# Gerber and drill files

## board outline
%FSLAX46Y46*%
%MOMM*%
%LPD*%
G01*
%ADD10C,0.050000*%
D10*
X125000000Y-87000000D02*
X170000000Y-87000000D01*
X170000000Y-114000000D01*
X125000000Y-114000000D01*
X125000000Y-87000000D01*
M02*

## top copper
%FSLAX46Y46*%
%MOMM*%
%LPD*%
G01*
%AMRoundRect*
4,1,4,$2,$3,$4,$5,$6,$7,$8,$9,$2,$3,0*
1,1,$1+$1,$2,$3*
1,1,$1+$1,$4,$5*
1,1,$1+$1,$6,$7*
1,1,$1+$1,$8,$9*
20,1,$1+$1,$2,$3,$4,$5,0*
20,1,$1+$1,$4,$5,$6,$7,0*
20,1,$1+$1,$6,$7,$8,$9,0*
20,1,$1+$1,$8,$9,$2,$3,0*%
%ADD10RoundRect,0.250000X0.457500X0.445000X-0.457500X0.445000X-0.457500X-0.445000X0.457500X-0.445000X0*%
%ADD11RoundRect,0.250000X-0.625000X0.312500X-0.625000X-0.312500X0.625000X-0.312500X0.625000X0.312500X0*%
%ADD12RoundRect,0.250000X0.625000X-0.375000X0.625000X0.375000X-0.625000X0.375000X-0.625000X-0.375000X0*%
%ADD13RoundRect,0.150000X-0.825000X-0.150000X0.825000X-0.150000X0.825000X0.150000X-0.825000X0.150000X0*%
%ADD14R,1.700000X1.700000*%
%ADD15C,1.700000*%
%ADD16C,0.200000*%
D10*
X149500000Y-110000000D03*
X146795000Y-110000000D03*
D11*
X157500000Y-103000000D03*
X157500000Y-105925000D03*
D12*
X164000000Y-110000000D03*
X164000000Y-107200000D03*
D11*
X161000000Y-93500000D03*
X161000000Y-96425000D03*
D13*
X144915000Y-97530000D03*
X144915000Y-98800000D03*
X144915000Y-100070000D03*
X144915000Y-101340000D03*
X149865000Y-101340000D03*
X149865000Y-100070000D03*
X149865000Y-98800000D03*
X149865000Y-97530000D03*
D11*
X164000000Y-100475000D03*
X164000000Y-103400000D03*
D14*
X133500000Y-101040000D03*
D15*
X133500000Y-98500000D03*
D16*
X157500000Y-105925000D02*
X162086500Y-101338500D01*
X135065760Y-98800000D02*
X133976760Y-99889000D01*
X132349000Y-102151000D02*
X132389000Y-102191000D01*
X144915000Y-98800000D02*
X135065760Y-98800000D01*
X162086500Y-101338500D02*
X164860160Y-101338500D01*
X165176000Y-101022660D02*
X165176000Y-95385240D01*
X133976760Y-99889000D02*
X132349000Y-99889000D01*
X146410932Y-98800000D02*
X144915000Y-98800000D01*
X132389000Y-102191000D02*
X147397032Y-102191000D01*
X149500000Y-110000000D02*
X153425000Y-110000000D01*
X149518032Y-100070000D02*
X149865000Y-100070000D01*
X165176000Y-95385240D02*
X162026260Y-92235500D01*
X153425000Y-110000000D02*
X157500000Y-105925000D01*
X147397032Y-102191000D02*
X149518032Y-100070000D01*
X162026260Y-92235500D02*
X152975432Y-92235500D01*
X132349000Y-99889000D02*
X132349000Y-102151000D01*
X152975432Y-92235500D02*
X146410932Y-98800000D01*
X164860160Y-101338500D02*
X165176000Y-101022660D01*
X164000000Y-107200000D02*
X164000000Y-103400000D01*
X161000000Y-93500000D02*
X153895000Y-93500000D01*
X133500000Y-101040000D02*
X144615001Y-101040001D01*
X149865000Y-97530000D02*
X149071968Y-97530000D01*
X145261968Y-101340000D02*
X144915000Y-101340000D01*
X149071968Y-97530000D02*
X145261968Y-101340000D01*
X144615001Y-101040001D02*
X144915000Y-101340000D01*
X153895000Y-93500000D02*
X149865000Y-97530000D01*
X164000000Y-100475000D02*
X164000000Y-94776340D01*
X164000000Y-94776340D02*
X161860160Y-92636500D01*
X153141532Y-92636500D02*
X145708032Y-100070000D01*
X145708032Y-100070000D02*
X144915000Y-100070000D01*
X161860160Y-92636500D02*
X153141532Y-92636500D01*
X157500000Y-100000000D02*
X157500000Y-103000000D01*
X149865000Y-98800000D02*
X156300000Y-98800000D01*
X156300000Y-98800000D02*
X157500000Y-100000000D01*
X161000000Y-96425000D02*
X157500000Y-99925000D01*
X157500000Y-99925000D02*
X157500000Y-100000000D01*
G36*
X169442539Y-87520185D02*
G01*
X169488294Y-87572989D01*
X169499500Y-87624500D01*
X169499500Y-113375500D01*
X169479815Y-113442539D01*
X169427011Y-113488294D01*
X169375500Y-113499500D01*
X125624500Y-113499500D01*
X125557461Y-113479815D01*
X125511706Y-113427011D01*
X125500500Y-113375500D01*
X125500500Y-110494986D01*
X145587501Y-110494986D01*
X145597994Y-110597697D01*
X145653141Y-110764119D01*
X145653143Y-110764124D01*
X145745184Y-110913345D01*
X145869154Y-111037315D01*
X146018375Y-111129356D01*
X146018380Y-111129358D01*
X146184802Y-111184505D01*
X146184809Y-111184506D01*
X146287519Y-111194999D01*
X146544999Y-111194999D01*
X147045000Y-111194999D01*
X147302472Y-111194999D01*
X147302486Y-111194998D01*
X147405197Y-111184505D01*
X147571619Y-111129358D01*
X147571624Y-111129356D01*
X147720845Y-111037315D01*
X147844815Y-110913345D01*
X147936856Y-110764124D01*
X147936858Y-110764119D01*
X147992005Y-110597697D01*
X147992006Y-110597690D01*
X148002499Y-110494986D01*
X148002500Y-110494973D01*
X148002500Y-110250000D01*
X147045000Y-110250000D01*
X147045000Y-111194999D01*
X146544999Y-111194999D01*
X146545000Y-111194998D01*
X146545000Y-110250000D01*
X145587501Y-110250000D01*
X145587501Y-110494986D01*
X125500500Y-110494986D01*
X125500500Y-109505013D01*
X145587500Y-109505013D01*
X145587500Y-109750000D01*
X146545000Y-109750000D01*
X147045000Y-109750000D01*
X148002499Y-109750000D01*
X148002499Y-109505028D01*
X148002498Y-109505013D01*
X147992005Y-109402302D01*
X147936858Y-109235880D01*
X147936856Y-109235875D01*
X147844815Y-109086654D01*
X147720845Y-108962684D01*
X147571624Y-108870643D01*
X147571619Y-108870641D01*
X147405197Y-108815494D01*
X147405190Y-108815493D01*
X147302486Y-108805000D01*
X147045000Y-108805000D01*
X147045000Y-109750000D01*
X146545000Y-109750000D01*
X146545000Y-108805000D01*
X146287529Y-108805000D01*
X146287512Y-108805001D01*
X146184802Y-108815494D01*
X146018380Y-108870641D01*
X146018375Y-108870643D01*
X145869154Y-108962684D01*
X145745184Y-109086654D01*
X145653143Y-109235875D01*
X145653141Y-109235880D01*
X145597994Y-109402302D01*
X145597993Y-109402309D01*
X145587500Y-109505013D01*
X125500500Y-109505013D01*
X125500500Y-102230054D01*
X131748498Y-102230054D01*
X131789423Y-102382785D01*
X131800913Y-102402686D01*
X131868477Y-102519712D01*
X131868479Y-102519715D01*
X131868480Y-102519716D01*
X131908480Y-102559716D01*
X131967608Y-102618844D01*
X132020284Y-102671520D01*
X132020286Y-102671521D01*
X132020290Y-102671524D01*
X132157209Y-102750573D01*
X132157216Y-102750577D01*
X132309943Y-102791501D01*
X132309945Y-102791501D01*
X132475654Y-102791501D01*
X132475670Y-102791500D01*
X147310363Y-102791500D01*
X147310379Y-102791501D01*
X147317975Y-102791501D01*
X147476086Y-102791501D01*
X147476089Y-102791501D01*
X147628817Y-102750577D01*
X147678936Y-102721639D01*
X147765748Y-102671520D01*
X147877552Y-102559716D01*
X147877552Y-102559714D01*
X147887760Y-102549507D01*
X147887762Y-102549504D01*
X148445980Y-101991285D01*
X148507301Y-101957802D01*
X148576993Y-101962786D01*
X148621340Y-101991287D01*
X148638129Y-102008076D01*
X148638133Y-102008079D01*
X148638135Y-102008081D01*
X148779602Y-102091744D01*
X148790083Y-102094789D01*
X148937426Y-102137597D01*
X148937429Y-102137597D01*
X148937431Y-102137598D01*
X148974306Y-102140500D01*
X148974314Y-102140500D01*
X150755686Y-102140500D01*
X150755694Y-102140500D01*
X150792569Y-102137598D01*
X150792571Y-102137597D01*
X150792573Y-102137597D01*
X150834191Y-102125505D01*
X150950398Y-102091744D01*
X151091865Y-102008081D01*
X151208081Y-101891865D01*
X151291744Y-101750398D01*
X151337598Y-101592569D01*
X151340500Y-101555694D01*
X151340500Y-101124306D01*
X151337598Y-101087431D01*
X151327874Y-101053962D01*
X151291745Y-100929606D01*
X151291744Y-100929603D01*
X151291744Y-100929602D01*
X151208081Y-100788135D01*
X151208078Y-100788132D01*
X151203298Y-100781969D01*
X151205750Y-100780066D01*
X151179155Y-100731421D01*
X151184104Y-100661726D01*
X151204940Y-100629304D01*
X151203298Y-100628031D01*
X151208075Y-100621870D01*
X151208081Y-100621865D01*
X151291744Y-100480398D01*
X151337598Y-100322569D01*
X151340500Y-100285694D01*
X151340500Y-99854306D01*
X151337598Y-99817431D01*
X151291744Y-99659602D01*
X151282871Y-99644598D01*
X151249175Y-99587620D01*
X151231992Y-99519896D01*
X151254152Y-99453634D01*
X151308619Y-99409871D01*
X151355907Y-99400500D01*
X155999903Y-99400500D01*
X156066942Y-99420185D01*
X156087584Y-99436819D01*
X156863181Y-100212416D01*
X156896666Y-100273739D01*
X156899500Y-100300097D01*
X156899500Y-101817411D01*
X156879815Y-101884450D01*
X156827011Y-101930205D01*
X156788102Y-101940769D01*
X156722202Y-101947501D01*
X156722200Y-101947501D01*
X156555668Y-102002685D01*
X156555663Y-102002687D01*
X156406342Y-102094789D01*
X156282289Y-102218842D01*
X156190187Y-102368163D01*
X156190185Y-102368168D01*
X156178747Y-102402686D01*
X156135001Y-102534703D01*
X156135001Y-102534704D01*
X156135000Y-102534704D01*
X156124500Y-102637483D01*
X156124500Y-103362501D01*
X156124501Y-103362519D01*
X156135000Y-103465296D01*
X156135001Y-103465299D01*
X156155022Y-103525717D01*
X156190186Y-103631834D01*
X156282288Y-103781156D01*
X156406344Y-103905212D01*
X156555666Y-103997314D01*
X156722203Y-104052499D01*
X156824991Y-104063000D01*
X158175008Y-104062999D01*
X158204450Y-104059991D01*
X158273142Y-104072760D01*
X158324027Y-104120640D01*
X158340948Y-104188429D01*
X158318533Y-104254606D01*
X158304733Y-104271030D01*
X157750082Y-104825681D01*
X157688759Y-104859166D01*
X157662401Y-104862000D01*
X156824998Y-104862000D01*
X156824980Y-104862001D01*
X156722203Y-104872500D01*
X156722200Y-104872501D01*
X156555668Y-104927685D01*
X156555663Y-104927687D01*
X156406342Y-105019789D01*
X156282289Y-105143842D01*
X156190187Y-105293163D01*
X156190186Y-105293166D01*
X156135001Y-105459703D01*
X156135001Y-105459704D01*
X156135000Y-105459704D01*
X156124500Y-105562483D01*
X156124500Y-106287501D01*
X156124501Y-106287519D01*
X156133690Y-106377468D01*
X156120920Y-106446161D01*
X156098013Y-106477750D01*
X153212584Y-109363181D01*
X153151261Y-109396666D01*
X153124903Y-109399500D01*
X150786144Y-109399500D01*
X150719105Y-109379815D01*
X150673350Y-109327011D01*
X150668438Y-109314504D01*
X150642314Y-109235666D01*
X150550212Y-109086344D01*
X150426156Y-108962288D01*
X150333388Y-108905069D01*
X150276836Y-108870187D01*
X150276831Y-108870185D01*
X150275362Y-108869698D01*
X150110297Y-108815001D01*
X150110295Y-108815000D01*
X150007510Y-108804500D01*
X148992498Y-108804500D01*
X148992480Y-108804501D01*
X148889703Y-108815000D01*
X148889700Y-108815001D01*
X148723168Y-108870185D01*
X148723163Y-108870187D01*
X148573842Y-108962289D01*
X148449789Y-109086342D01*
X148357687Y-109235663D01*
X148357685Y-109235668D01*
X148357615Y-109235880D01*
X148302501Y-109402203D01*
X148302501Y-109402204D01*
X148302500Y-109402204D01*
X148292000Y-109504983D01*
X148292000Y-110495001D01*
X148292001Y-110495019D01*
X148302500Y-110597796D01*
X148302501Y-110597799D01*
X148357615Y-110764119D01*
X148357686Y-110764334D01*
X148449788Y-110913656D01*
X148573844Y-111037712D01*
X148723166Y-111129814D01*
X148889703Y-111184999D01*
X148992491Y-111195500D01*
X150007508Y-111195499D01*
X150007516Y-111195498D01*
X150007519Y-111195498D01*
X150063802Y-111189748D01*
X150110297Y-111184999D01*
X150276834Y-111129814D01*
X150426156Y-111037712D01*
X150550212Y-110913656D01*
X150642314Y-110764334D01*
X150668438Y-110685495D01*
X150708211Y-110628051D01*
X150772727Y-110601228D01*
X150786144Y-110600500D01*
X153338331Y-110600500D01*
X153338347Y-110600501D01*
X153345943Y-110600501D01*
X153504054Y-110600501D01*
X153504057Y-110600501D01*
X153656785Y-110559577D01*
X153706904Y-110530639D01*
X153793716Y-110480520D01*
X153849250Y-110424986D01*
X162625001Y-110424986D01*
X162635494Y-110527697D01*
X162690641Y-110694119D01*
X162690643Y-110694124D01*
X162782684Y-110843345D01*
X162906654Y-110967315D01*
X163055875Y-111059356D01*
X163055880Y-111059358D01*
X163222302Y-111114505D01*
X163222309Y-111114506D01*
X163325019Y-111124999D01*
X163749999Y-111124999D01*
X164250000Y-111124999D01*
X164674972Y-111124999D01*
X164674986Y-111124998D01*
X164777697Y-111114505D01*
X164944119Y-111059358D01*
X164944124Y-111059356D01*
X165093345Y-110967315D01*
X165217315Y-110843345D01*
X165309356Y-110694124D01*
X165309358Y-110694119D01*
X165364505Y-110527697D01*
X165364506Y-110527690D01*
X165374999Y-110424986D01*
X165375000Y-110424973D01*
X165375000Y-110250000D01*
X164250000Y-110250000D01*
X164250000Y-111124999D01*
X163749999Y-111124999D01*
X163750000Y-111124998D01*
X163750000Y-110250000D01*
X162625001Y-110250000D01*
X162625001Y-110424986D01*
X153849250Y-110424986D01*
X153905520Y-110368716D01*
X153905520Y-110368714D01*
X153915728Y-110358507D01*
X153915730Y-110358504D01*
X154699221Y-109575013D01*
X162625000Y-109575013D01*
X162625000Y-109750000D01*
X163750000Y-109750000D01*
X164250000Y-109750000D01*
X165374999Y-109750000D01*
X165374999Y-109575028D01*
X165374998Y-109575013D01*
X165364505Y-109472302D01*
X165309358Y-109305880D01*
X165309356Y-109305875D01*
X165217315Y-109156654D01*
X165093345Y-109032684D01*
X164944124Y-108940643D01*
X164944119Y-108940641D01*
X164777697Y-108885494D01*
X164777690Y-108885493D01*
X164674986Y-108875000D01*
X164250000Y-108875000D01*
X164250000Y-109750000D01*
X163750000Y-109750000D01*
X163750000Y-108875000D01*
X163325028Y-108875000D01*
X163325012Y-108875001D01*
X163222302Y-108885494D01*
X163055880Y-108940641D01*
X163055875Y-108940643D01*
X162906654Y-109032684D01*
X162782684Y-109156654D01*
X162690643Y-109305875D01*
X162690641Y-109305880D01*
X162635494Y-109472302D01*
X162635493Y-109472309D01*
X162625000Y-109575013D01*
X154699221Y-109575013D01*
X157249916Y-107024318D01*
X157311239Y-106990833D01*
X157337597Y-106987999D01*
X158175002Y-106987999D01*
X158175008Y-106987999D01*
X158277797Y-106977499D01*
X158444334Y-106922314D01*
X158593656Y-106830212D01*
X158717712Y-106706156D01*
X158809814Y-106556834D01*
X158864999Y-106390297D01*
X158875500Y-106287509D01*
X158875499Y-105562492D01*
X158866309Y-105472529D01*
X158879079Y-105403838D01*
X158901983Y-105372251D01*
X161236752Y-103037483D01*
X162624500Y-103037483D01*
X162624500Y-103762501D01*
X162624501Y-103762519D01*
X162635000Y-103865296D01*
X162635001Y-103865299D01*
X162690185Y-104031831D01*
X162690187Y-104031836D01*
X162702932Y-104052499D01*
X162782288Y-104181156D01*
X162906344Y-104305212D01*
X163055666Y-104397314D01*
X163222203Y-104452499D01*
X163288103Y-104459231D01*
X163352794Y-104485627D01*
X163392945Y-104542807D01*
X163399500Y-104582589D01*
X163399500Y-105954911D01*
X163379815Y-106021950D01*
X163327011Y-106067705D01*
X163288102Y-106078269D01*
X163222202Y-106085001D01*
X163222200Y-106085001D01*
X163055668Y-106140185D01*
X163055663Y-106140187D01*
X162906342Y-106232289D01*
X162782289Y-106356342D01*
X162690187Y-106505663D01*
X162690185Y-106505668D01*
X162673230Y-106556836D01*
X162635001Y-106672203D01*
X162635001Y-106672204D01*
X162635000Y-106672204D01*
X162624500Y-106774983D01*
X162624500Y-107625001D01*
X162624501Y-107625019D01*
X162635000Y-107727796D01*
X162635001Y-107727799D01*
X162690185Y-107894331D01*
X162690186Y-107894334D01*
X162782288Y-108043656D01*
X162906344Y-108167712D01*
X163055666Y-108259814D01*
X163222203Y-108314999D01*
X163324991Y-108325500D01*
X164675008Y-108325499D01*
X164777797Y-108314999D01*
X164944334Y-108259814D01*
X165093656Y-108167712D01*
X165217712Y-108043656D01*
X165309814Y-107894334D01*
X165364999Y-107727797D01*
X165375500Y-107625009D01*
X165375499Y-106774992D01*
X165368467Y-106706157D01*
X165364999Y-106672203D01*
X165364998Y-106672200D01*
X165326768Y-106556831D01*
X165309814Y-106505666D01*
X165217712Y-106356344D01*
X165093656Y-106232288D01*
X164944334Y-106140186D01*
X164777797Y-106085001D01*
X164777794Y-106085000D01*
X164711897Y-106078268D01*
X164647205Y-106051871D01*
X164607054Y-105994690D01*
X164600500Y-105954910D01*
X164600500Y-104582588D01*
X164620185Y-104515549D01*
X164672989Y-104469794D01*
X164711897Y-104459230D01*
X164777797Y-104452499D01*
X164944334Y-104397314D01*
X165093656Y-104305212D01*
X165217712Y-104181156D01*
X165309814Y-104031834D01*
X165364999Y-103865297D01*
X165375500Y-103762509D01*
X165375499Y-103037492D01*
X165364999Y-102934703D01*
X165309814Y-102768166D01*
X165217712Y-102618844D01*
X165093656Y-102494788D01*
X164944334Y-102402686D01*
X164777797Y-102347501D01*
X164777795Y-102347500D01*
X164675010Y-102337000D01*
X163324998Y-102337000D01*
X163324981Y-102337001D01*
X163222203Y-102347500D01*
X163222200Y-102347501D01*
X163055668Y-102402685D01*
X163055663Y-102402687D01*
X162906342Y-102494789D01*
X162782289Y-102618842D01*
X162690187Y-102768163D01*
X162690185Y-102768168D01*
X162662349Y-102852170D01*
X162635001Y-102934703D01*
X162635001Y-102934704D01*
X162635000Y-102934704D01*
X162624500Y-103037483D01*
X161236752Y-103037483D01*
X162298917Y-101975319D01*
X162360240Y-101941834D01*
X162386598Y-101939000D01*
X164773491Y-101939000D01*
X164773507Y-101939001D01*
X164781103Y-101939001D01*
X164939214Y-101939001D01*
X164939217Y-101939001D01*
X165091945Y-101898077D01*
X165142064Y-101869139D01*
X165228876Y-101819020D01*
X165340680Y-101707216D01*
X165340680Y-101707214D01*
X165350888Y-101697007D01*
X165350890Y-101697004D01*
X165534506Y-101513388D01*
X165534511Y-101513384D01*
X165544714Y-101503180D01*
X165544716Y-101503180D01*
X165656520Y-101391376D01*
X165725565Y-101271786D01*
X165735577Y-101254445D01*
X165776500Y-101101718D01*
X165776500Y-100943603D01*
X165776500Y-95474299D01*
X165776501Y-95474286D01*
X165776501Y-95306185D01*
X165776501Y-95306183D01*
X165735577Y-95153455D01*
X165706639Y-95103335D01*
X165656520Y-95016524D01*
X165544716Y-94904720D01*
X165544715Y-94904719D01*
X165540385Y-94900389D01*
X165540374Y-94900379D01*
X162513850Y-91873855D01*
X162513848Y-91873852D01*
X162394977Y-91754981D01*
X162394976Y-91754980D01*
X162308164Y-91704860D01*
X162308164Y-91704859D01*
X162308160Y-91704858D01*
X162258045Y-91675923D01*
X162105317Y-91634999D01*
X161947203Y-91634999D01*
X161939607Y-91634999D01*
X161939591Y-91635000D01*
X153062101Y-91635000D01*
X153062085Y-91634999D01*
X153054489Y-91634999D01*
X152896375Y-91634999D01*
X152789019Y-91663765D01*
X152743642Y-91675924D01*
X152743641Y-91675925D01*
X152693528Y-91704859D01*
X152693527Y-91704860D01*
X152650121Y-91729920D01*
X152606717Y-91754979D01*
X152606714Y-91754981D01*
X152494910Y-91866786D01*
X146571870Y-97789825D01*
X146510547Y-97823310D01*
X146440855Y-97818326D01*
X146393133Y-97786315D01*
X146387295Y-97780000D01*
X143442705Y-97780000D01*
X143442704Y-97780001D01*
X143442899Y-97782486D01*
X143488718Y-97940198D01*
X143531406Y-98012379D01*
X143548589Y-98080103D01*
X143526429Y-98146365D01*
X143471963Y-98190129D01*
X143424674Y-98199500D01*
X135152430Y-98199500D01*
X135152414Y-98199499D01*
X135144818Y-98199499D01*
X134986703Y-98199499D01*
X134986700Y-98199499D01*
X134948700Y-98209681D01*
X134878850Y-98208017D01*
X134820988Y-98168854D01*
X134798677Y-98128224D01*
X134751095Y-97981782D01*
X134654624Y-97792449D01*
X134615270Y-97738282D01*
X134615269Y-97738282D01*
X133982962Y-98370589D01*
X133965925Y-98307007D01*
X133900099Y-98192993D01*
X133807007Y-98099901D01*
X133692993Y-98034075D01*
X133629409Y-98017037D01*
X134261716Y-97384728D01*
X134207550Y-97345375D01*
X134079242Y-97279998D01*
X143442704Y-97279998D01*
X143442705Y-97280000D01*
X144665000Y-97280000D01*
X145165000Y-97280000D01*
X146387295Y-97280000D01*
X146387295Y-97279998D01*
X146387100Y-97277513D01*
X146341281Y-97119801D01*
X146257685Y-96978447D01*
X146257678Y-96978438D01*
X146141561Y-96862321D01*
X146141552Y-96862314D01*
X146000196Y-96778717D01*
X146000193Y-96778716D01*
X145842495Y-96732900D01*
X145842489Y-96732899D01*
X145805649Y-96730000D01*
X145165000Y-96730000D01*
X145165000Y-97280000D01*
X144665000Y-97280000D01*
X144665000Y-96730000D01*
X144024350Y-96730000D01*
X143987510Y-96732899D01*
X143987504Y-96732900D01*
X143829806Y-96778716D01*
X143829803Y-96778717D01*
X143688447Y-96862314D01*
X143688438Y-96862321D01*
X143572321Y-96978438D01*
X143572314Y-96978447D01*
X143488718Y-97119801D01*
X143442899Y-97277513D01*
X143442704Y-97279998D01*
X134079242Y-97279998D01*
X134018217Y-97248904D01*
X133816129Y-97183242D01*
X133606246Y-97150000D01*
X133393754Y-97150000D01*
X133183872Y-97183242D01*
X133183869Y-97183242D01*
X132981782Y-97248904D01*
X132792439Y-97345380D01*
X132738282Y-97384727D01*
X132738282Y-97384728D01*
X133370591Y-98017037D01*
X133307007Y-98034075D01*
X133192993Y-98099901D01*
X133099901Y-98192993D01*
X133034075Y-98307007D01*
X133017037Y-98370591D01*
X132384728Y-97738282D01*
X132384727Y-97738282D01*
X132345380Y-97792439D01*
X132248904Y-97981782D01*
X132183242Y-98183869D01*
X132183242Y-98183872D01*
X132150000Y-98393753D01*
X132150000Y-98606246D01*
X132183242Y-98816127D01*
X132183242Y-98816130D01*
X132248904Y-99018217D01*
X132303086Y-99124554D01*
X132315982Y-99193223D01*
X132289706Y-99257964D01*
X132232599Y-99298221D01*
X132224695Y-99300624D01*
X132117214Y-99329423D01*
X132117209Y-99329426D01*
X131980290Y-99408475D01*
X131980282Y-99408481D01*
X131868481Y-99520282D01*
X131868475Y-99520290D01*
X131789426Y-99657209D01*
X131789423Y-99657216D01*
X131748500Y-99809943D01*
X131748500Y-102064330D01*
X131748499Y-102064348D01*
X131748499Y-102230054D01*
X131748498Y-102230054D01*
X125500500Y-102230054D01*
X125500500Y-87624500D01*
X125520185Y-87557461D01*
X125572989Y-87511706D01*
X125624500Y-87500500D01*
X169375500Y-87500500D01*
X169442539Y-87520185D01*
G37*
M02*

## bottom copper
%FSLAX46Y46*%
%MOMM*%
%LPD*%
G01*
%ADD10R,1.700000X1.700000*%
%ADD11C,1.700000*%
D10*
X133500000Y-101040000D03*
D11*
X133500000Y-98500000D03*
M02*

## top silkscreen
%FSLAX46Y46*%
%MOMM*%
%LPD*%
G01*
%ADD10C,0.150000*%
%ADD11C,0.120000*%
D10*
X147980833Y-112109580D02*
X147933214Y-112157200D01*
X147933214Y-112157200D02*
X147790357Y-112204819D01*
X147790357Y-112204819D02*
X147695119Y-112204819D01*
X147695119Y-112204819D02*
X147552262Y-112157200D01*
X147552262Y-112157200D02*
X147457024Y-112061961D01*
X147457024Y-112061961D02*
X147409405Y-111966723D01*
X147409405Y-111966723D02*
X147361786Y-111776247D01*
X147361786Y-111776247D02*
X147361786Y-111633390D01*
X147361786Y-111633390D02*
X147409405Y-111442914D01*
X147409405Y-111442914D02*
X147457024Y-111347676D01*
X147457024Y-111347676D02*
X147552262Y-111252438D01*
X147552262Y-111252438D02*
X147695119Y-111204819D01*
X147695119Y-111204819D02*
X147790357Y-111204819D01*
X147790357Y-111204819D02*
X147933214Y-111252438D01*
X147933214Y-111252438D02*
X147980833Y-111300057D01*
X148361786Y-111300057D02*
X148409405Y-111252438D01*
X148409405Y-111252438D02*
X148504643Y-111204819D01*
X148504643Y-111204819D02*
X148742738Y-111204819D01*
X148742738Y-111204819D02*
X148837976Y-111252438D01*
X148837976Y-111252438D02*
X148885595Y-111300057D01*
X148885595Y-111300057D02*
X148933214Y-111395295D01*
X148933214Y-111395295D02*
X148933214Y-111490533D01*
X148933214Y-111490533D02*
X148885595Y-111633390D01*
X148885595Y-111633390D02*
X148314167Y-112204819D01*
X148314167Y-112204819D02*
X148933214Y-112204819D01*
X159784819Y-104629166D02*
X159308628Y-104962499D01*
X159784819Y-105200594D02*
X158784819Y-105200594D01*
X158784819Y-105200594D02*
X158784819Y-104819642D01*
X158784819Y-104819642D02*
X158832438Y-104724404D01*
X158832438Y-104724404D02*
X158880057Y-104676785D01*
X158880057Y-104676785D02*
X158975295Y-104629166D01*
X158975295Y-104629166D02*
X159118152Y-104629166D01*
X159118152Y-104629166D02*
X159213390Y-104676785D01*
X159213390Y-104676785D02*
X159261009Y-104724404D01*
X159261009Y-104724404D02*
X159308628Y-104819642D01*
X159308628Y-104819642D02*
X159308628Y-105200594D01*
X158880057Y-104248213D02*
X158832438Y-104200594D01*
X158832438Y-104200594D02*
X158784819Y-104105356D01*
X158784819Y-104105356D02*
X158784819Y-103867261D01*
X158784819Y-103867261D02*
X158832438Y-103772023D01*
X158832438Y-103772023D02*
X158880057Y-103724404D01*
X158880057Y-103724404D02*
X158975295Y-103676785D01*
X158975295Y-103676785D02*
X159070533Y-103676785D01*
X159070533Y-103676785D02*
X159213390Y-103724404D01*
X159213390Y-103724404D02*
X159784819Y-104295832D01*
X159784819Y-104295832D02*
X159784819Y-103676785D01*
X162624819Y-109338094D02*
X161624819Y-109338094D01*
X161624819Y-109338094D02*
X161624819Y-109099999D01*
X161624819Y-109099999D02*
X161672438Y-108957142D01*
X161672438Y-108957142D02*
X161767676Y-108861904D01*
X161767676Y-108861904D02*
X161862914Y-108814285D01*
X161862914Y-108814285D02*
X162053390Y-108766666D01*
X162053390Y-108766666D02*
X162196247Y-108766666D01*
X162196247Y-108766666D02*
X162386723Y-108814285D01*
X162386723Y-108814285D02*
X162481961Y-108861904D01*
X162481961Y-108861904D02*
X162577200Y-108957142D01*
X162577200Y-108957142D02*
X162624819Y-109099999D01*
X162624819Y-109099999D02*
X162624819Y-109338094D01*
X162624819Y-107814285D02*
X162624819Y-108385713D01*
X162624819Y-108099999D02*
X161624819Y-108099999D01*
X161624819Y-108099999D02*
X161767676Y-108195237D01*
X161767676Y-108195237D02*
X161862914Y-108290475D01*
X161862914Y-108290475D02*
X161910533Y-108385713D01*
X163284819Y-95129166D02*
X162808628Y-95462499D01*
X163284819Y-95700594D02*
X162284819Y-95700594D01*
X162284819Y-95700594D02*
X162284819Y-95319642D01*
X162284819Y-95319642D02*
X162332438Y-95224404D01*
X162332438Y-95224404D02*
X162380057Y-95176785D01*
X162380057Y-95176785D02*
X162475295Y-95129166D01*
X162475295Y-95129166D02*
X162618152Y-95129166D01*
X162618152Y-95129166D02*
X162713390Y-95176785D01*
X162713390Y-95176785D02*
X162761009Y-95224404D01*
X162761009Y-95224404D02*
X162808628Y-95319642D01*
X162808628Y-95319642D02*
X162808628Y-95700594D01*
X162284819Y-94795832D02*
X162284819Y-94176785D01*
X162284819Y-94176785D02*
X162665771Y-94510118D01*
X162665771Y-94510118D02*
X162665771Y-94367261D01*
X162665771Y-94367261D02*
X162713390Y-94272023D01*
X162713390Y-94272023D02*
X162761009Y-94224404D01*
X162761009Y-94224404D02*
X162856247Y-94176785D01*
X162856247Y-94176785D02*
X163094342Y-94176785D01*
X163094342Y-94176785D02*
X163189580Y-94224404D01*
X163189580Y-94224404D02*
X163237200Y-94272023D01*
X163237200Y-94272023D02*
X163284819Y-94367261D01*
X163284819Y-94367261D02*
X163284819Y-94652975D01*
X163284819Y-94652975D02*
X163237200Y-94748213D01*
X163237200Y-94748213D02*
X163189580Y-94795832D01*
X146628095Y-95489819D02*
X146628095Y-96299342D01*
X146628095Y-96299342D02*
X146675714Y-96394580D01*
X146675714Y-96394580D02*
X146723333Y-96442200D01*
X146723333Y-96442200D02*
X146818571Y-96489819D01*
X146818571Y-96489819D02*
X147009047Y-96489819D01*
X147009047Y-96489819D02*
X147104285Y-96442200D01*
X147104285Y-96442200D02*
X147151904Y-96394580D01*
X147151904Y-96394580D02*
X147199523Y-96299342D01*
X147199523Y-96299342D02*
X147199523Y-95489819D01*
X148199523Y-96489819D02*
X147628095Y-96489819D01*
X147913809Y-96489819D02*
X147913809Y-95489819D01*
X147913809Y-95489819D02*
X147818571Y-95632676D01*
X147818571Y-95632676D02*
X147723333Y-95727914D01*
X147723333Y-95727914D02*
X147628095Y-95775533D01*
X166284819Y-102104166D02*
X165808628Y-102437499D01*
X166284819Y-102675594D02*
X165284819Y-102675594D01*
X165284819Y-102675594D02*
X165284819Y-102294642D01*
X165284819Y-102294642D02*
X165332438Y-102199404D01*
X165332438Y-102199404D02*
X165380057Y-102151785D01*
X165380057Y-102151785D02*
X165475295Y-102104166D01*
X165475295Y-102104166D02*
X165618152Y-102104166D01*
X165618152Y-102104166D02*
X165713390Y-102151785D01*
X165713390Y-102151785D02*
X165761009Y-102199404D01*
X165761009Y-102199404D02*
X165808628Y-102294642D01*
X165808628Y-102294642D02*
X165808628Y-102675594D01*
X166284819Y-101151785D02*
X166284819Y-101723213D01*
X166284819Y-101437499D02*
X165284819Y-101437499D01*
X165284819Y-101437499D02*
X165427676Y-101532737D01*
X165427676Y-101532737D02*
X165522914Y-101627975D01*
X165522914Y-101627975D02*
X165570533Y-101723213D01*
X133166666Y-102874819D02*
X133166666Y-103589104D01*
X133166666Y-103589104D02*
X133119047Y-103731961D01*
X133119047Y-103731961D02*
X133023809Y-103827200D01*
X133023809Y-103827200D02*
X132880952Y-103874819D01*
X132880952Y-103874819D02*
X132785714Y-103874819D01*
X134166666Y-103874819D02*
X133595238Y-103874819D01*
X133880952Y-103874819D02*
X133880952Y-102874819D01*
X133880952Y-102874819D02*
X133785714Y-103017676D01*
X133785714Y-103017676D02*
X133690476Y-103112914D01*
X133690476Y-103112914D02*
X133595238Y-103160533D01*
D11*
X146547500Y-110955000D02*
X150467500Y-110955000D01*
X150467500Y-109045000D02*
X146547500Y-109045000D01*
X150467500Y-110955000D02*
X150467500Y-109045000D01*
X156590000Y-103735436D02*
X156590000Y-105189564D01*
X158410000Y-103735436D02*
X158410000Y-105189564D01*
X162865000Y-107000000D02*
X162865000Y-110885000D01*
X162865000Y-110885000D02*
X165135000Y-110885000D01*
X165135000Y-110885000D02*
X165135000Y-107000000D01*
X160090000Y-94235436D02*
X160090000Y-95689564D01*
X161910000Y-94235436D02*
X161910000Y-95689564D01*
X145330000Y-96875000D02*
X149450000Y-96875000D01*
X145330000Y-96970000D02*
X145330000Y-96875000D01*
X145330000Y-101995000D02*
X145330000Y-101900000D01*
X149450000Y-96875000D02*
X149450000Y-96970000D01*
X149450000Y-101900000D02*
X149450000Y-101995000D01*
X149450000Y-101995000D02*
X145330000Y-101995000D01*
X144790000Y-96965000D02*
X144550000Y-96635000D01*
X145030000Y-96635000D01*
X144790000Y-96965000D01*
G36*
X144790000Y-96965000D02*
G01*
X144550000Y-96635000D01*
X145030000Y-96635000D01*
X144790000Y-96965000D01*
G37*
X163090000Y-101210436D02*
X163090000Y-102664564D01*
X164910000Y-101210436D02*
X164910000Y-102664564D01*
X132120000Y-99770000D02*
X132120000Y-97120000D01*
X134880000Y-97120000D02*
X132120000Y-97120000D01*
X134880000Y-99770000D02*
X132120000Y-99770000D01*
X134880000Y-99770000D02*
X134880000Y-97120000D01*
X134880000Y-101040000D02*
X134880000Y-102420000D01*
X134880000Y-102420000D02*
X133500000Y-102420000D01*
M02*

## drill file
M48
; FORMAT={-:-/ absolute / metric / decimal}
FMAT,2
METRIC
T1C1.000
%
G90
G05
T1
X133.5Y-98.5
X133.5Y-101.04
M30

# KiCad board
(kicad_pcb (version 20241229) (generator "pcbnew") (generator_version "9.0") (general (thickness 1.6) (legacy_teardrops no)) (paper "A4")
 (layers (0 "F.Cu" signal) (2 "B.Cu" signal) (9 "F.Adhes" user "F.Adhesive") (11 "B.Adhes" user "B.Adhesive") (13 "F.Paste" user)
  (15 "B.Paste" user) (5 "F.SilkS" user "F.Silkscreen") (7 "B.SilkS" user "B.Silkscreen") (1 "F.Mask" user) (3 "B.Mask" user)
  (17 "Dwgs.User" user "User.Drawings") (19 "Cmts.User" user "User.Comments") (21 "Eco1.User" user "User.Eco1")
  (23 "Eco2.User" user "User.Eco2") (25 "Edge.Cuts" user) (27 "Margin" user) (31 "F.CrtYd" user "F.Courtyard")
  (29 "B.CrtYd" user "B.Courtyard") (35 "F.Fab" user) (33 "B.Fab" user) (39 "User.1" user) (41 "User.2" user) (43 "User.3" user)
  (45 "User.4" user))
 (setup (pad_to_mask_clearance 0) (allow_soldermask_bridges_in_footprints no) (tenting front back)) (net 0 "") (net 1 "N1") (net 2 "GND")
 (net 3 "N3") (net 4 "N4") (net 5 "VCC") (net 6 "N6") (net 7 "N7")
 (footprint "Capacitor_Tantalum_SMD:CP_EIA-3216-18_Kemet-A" (layer "F.Cu") (at 148.1475 110 180)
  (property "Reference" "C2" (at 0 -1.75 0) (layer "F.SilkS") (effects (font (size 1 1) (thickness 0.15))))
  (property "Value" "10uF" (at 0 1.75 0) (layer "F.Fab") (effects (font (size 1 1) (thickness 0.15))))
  (fp_line (start 1.6 -0.955) (end -2.32 -0.955) (stroke (width 0.12) (type solid)) (layer "F.SilkS"))
  (fp_line (start -2.32 0.955) (end 1.6 0.955) (stroke (width 0.12) (type solid)) (layer "F.SilkS"))
  (fp_line (start -2.32 -0.955) (end -2.32 0.955) (stroke (width 0.12) (type solid)) (layer "F.SilkS"))
  (pad "1" smd roundrect (at -1.3525 0 180) (size 1.415 1.39) (layers "F.Cu" "F.Mask" "F.Paste") (roundrect_rratio 0.179856) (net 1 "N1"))
  (pad "2" smd roundrect (at 1.3525 0 180) (size 1.415 1.39) (layers "F.Cu" "F.Mask" "F.Paste") (roundrect_rratio 0.179856) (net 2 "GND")))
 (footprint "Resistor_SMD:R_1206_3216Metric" (layer "F.Cu") (at 157.5 104.4625 -90)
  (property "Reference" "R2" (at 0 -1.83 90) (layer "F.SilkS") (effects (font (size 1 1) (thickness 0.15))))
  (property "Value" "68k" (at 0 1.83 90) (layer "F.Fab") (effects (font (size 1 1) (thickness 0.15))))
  (fp_line (start -0.727064 0.91) (end 0.727064 0.91) (stroke (width 0.12) (type solid)) (layer "F.SilkS"))
  (fp_line (start -0.727064 -0.91) (end 0.727064 -0.91) (stroke (width 0.12) (type solid)) (layer "F.SilkS"))
  (pad "1" smd roundrect (at -1.4625 0 270) (size 1.125 1.75) (layers "F.Cu" "F.Mask" "F.Paste") (roundrect_rratio 0.222222) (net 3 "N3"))
  (pad "2" smd roundrect (at 1.4625 0 270) (size 1.125 1.75) (layers "F.Cu" "F.Mask" "F.Paste") (roundrect_rratio 0.222222) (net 1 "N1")))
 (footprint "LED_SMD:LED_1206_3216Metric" (layer "F.Cu") (at 164 108.6 90)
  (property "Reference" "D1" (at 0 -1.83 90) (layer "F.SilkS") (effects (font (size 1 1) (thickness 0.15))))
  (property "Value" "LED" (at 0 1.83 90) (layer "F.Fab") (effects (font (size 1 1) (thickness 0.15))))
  (fp_line (start 1.6 -1.135) (end -2.285 -1.135) (stroke (width 0.12) (type solid)) (layer "F.SilkS"))
  (fp_line (start -2.285 -1.135) (end -2.285 1.135) (stroke (width 0.12) (type solid)) (layer "F.SilkS"))
  (fp_line (start -2.285 1.135) (end 1.6 1.135) (stroke (width 0.12) (type solid)) (layer "F.SilkS"))
  (pad "1" smd roundrect (at -1.4 0 90) (size 1.25 1.75) (layers "F.Cu" "F.Mask" "F.Paste") (roundrect_rratio 0.2) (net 2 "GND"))
  (pad "2" smd roundrect (at 1.4 0 90) (size 1.25 1.75) (layers "F.Cu" "F.Mask" "F.Paste") (roundrect_rratio 0.2) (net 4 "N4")))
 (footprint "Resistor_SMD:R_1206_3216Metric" (layer "F.Cu") (at 161 94.9625 -90)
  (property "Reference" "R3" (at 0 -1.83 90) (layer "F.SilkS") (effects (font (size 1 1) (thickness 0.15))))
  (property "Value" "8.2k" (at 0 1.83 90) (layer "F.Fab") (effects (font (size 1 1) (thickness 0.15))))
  (fp_line (start -0.727064 0.91) (end 0.727064 0.91) (stroke (width 0.12) (type solid)) (layer "F.SilkS"))
  (fp_line (start -0.727064 -0.91) (end 0.727064 -0.91) (stroke (width 0.12) (type solid)) (layer "F.SilkS"))
  (pad "1" smd roundrect (at -1.4625 0 270) (size 1.125 1.75) (layers "F.Cu" "F.Mask" "F.Paste") (roundrect_rratio 0.222222) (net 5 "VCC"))
  (pad "2" smd roundrect (at 1.4625 0 270) (size 1.125 1.75) (layers "F.Cu" "F.Mask" "F.Paste") (roundrect_rratio 0.222222) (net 3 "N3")))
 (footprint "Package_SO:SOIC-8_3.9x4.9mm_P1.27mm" (layer "F.Cu") (at 147.39 99.435)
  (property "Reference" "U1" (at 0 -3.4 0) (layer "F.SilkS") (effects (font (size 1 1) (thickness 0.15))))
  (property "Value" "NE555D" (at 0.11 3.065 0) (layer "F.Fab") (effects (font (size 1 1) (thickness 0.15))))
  (fp_line (start -2.06 -2.56) (end 2.06 -2.56) (stroke (width 0.12) (type solid)) (layer "F.SilkS"))
  (fp_line (start -2.06 -2.465) (end -2.06 -2.56) (stroke (width 0.12) (type solid)) (layer "F.SilkS"))
  (fp_line (start -2.06 2.56) (end -2.06 2.465) (stroke (width 0.12) (type solid)) (layer "F.SilkS"))
  (fp_line (start 2.06 -2.56) (end 2.06 -2.465) (stroke (width 0.12) (type solid)) (layer "F.SilkS"))
  (fp_line (start 2.06 2.465) (end 2.06 2.56) (stroke (width 0.12) (type solid)) (layer "F.SilkS"))
  (fp_line (start 2.06 2.56) (end -2.06 2.56) (stroke (width 0.12) (type solid)) (layer "F.SilkS"))
  (fp_poly (pts (xy -2.6 -2.47) (xy -2.84 -2.8) (xy -2.36 -2.8)) (stroke (width 0.12) (type solid)) (fill yes) (layer "F.SilkS"))
  (pad "1" smd roundrect (at -2.475 -1.905) (size 1.95 0.6) (layers "F.Cu" "F.Mask" "F.Paste") (roundrect_rratio 0.25) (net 2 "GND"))
  (pad "2" smd roundrect (at -2.475 -0.635) (size 1.95 0.6) (layers "F.Cu" "F.Mask" "F.Paste") (roundrect_rratio 0.25) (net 1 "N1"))
  (pad "3" smd roundrect (at -2.475 0.635) (size 1.95 0.6) (layers "F.Cu" "F.Mask" "F.Paste") (roundrect_rratio 0.25) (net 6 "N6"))
  (pad "4" smd roundrect (at -2.475 1.905) (size 1.95 0.6) (layers "F.Cu" "F.Mask" "F.Paste") (roundrect_rratio 0.25) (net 5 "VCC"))
  (pad "5" smd roundrect (at 2.475 1.905) (size 1.95 0.6) (layers "F.Cu" "F.Mask" "F.Paste") (roundrect_rratio 0.25) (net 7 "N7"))
  (pad "6" smd roundrect (at 2.475 0.635) (size 1.95 0.6) (layers "F.Cu" "F.Mask" "F.Paste") (roundrect_rratio 0.25) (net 1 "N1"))
  (pad "7" smd roundrect (at 2.475 -0.635) (size 1.95 0.6) (layers "F.Cu" "F.Mask" "F.Paste") (roundrect_rratio 0.25) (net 3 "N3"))
  (pad "8" smd roundrect (at 2.475 -1.905) (size 1.95 0.6) (layers "F.Cu" "F.Mask" "F.Paste") (roundrect_rratio 0.25) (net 5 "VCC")))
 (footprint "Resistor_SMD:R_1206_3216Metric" (layer "F.Cu") (at 164 101.9375 -90)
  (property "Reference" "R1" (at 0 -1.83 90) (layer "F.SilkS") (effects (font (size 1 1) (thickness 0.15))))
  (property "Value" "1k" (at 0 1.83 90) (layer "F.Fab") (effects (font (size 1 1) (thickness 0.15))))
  (fp_line (start -0.727064 0.91) (end 0.727064 0.91) (stroke (width 0.12) (type solid)) (layer "F.SilkS"))
  (fp_line (start -0.727064 -0.91) (end 0.727064 -0.91) (stroke (width 0.12) (type solid)) (layer "F.SilkS"))
  (pad "1" smd roundrect (at -1.4625 0 270) (size 1.125 1.75) (layers "F.Cu" "F.Mask" "F.Paste") (roundrect_rratio 0.222222) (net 6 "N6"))
  (pad "2" smd roundrect (at 1.4625 0 270) (size 1.125 1.75) (layers "F.Cu" "F.Mask" "F.Paste") (roundrect_rratio 0.222222) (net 4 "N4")))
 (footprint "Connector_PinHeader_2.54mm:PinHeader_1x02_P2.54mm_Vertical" (layer "F.Cu") (at 133.5 101.04 180)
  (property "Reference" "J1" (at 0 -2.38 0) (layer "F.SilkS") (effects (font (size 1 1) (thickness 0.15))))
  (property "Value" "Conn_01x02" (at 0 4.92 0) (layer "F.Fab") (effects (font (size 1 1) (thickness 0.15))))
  (fp_line (start 1.38 1.27) (end 1.38 3.92) (stroke (width 0.12) (type solid)) (layer "F.SilkS"))
  (fp_line (start -1.38 3.92) (end 1.38 3.92) (stroke (width 0.12) (type solid)) (layer "F.SilkS"))
  (fp_line (start -1.38 1.27) (end 1.38 1.27) (stroke (width 0.12) (type solid)) (layer "F.SilkS"))
  (fp_line (start -1.38 1.27) (end -1.38 3.92) (stroke (width 0.12) (type solid)) (layer "F.SilkS"))
  (fp_line (start -1.38 0) (end -1.38 -1.38) (stroke (width 0.12) (type solid)) (layer "F.SilkS"))
  (fp_line (start -1.38 -1.38) (end 0 -1.38) (stroke (width 0.12) (type solid)) (layer "F.SilkS"))
  (pad "1" thru_hole rect (at 0 0 180) (size 1.7 1.7) (drill 1) (layers "*.Cu" "*.Mask") (remove_unused_layers no) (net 5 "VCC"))
  (pad "2" thru_hole circle (at 0 2.54 180) (size 1.7 1.7) (drill 1) (layers "*.Cu" "*.Mask") (remove_unused_layers no) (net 2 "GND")))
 (gr_rect (start 125 87) (end 170 114) (stroke (width 0.05) (type default)) (fill no) (layer "Edge.Cuts"))
 (segment (start 157.5 105.925) (end 162.0865 101.3385) (width 0.2) (layer "F.Cu") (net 1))
 (segment (start 135.06576 98.8) (end 133.97676 99.889) (width 0.2) (layer "F.Cu") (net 1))
 (segment (start 132.349 102.151) (end 132.389 102.191) (width 0.2) (layer "F.Cu") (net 1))
 (segment (start 144.915 98.8) (end 135.06576 98.8) (width 0.2) (layer "F.Cu") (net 1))
 (segment (start 162.0865 101.3385) (end 164.86016 101.3385) (width 0.2) (layer "F.Cu") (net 1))
 (segment (start 165.176 101.02266) (end 165.176 95.38524) (width 0.2) (layer "F.Cu") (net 1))
 (segment (start 133.97676 99.889) (end 132.349 99.889) (width 0.2) (layer "F.Cu") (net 1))
 (segment (start 146.410932 98.8) (end 144.915 98.8) (width 0.2) (layer "F.Cu") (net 1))
 (segment (start 132.389 102.191) (end 147.397032 102.191) (width 0.2) (layer "F.Cu") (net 1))
 (segment (start 149.5 110) (end 153.425 110) (width 0.2) (layer "F.Cu") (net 1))
 (segment (start 149.518032 100.07) (end 149.865 100.07) (width 0.2) (layer "F.Cu") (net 1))
 (segment (start 165.176 95.38524) (end 162.02626 92.2355) (width 0.2) (layer "F.Cu") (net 1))
 (segment (start 153.425 110) (end 157.5 105.925) (width 0.2) (layer "F.Cu") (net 1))
 (segment (start 147.397032 102.191) (end 149.518032 100.07) (width 0.2) (layer "F.Cu") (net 1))
 (segment (start 162.02626 92.2355) (end 152.975432 92.2355) (width 0.2) (layer "F.Cu") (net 1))
 (segment (start 132.349 99.889) (end 132.349 102.151) (width 0.2) (layer "F.Cu") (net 1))
 (segment (start 152.975432 92.2355) (end 146.410932 98.8) (width 0.2) (layer "F.Cu") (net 1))
 (segment (start 164.86016 101.3385) (end 165.176 101.02266) (width 0.2) (layer "F.Cu") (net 1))
 (segment (start 164 107.2) (end 164 103.4) (width 0.2) (layer "F.Cu") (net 4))
 (segment (start 161 93.5) (end 153.895 93.5) (width 0.2) (layer "F.Cu") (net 5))
 (segment (start 133.5 101.04) (end 144.615001 101.040001) (width 0.2) (layer "F.Cu") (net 5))
 (segment (start 149.865 97.53) (end 149.071968 97.53) (width 0.2) (layer "F.Cu") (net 5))
 (segment (start 145.261968 101.34) (end 144.915 101.34) (width 0.2) (layer "F.Cu") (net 5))
 (segment (start 149.071968 97.53) (end 145.261968 101.34) (width 0.2) (layer "F.Cu") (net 5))
 (segment (start 144.615001 101.040001) (end 144.915 101.34) (width 0.2) (layer "F.Cu") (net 5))
 (segment (start 153.895 93.5) (end 149.865 97.53) (width 0.2) (layer "F.Cu") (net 5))
 (segment (start 164 100.475) (end 164 94.77634) (width 0.2) (layer "F.Cu") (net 6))
 (segment (start 164 94.77634) (end 161.86016 92.6365) (width 0.2) (layer "F.Cu") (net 6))
 (segment (start 153.141532 92.6365) (end 145.708032 100.07) (width 0.2) (layer "F.Cu") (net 6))
 (segment (start 145.708032 100.07) (end 144.915 100.07) (width 0.2) (layer "F.Cu") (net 6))
 (segment (start 161.86016 92.6365) (end 153.141532 92.6365) (width 0.2) (layer "F.Cu") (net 6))
 (segment (start 157.5 100) (end 157.5 103) (width 0.2) (layer "F.Cu") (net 3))
 (segment (start 149.865 98.8) (end 156.3 98.8) (width 0.2) (layer "F.Cu") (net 3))
 (segment (start 156.3 98.8) (end 157.5 100) (width 0.2) (layer "F.Cu") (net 3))
 (segment (start 161 96.425) (end 157.5 99.925) (width 0.2) (layer "F.Cu") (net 3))
 (segment (start 157.5 99.925) (end 157.5 100) (width 0.2) (layer "F.Cu") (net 3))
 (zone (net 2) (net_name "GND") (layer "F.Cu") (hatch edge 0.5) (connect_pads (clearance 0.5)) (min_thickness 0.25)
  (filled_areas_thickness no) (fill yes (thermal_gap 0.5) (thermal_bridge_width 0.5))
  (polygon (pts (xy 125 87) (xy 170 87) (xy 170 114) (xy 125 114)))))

